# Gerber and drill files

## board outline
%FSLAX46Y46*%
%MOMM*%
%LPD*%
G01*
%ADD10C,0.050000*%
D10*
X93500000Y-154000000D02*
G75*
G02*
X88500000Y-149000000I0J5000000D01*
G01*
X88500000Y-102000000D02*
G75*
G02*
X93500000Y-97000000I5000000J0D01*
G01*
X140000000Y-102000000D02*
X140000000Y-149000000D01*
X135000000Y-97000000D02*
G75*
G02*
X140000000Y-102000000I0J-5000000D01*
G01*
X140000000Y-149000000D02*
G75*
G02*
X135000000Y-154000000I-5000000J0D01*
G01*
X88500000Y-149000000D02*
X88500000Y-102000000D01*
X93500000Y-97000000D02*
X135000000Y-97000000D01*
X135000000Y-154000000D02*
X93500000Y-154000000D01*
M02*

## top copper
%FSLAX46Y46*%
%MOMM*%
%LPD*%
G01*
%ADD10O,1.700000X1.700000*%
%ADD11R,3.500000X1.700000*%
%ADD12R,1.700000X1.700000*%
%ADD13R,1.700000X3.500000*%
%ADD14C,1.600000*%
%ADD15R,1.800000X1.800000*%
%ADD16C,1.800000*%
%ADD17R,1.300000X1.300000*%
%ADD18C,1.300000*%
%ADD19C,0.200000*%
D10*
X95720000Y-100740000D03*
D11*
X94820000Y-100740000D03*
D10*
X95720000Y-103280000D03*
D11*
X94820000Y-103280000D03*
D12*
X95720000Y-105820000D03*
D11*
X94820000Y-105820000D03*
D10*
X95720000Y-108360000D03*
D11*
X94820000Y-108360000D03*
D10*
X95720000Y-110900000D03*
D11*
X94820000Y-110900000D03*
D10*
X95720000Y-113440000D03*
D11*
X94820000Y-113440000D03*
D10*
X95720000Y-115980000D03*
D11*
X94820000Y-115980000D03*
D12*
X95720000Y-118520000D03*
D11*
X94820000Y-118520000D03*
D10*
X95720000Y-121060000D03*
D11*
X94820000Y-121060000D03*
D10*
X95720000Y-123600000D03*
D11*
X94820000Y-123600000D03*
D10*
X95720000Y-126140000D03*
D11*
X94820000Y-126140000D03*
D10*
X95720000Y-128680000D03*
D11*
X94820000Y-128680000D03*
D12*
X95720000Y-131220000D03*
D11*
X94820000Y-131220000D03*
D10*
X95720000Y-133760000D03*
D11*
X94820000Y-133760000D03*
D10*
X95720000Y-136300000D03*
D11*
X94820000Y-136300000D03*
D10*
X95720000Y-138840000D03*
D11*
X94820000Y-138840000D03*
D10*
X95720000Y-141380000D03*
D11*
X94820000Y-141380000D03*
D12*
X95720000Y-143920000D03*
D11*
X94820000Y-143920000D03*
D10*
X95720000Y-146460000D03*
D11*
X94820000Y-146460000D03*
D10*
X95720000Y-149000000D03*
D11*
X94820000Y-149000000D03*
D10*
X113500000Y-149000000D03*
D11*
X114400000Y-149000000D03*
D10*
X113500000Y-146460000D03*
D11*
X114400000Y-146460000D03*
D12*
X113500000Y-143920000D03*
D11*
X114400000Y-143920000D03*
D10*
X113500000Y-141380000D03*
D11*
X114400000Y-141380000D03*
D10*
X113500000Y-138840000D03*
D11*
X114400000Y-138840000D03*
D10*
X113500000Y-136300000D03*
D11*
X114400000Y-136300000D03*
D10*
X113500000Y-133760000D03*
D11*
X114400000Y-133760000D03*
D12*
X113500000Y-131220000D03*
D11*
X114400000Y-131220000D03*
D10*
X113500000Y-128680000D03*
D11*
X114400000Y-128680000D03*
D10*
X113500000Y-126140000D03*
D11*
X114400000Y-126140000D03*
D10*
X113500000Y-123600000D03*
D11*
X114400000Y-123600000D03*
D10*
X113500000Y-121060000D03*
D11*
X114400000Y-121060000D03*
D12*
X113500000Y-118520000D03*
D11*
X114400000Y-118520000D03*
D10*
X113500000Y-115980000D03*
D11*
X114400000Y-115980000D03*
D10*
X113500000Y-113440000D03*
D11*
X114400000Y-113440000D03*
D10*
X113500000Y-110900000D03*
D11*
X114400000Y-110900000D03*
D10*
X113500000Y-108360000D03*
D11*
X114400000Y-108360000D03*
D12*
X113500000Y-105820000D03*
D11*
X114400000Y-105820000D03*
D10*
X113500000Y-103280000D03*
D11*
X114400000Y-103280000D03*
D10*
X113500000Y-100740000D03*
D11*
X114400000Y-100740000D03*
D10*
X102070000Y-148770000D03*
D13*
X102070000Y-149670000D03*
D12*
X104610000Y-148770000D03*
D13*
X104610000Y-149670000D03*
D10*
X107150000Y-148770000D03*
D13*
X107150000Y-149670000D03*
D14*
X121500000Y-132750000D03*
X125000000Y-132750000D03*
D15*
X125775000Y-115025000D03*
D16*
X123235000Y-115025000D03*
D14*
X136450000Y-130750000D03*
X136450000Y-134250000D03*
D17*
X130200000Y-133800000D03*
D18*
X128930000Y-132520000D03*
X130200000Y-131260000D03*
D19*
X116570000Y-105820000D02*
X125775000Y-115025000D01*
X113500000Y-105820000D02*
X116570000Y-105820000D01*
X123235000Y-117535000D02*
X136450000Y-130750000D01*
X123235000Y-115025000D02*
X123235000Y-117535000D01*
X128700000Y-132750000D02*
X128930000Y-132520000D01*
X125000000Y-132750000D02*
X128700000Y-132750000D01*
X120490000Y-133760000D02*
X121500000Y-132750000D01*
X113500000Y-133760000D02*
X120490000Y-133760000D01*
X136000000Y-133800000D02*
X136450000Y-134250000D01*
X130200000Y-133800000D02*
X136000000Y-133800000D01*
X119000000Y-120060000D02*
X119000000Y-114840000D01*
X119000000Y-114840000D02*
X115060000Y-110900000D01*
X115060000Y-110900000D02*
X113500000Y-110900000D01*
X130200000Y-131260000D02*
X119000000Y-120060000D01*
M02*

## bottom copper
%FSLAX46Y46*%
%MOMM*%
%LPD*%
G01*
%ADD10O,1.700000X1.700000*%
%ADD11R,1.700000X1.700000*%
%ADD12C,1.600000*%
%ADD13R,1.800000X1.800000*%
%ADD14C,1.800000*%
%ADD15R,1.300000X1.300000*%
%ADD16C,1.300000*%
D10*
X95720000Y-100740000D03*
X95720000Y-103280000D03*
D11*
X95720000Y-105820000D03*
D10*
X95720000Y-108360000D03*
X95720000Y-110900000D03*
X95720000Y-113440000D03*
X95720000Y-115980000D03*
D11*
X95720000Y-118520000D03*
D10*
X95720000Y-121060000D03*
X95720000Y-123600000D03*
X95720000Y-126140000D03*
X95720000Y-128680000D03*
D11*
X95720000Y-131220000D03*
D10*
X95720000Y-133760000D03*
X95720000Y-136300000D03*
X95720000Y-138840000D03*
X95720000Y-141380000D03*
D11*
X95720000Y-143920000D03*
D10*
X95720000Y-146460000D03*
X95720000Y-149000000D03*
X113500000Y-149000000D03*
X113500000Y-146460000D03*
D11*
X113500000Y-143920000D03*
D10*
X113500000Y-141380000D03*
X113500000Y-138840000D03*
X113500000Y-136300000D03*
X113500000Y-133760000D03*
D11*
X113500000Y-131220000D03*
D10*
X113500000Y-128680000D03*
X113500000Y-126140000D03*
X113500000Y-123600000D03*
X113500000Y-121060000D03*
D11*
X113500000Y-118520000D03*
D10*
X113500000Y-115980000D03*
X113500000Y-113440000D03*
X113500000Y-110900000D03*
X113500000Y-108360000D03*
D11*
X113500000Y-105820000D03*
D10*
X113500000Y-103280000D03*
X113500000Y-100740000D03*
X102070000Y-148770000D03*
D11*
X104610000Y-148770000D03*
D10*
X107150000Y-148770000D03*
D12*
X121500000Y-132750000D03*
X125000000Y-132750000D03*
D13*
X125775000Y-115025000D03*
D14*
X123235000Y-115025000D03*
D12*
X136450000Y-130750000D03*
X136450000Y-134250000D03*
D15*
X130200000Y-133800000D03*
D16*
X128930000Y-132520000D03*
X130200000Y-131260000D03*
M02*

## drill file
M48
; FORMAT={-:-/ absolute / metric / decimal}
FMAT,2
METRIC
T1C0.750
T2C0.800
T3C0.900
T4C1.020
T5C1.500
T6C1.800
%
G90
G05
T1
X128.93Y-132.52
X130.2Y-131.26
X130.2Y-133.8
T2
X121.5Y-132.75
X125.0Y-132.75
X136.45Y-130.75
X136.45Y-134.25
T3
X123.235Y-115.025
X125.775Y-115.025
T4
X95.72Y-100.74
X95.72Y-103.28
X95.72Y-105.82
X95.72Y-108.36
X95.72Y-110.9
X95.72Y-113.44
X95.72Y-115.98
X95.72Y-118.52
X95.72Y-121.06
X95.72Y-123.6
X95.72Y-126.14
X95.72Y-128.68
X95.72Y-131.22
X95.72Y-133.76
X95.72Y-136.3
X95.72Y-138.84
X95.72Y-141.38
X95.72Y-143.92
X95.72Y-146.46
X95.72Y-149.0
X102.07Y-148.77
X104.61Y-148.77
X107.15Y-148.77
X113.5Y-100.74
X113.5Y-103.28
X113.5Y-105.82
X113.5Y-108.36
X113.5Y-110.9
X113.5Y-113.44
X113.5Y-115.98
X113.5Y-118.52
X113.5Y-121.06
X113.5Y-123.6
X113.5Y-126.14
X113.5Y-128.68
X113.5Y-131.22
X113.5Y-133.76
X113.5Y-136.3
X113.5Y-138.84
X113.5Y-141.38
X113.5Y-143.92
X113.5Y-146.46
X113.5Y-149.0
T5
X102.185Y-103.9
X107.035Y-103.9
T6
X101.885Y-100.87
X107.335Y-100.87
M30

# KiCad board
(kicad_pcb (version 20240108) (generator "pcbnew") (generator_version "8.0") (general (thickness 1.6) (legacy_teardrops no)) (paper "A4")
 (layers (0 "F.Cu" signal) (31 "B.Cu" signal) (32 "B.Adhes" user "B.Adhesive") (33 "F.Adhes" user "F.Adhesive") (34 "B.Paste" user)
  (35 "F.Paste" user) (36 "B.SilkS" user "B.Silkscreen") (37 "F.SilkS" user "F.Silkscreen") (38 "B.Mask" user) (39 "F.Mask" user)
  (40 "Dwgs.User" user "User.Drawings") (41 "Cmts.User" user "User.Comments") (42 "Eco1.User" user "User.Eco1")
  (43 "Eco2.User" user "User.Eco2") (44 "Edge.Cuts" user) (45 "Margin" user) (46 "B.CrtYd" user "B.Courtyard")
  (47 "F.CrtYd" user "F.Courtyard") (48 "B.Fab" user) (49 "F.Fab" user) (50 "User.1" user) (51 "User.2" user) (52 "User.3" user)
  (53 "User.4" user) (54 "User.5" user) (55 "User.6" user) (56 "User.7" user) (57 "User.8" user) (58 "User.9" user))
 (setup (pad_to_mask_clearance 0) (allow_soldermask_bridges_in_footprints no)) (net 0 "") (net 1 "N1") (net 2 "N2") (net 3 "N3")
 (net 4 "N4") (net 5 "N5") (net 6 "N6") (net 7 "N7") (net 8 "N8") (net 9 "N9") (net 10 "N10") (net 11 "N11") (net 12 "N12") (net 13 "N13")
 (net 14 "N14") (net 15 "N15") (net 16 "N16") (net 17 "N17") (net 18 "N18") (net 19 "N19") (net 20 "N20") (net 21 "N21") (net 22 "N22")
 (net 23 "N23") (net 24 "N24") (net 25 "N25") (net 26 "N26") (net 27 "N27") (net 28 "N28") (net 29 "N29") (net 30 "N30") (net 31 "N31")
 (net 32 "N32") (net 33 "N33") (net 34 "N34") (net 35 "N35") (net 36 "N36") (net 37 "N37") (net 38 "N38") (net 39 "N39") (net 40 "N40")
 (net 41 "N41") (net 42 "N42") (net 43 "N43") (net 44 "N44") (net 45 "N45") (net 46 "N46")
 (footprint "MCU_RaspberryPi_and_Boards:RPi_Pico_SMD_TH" (layer "F.Cu") (at 104.61 124.87)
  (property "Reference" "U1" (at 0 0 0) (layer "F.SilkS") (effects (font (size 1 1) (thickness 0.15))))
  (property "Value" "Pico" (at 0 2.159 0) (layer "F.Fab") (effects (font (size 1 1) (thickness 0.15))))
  (pad "" np_thru_hole oval (at -2.725 -24) (size 1.8 1.8) (drill 1.8) (layers "*.Cu" "*.Mask"))
  (pad "" np_thru_hole oval (at -2.425 -20.97) (size 1.5 1.5) (drill 1.5) (layers "*.Cu" "*.Mask"))
  (pad "" np_thru_hole oval (at 2.425 -20.97) (size 1.5 1.5) (drill 1.5) (layers "*.Cu" "*.Mask"))
  (pad "" np_thru_hole oval (at 2.725 -24) (size 1.8 1.8) (drill 1.8) (layers "*.Cu" "*.Mask"))
  (pad "1" thru_hole oval (at -8.89 -24.13) (size 1.7 1.7) (drill 1.02) (layers "*.Cu" "*.Mask") (remove_unused_layers no) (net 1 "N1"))
  (pad "1" smd rect (at -8.89 -24.13) (size 3.5 1.7) (drill (offset -0.9 0)) (layers "F.Cu" "F.Mask") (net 1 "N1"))
  (pad "2" thru_hole oval (at -8.89 -21.59) (size 1.7 1.7) (drill 1.02) (layers "*.Cu" "*.Mask") (remove_unused_layers no) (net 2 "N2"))
  (pad "2" smd rect (at -8.89 -21.59) (size 3.5 1.7) (drill (offset -0.9 0)) (layers "F.Cu" "F.Mask") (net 2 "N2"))
  (pad "3" thru_hole rect (at -8.89 -19.05) (size 1.7 1.7) (drill 1.02) (layers "*.Cu" "*.Mask") (remove_unused_layers no) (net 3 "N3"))
  (pad "3" smd rect (at -8.89 -19.05) (size 3.5 1.7) (drill (offset -0.9 0)) (layers "F.Cu" "F.Mask") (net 3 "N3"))
  (pad "4" thru_hole oval (at -8.89 -16.51) (size 1.7 1.7) (drill 1.02) (layers "*.Cu" "*.Mask") (remove_unused_layers no) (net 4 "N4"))
  (pad "4" smd rect (at -8.89 -16.51) (size 3.5 1.7) (drill (offset -0.9 0)) (layers "F.Cu" "F.Mask") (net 4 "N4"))
  (pad "5" thru_hole oval (at -8.89 -13.97) (size 1.7 1.7) (drill 1.02) (layers "*.Cu" "*.Mask") (remove_unused_layers no) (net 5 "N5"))
  (pad "5" smd rect (at -8.89 -13.97) (size 3.5 1.7) (drill (offset -0.9 0)) (layers "F.Cu" "F.Mask") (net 5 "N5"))
  (pad "6" thru_hole oval (at -8.89 -11.43) (size 1.7 1.7) (drill 1.02) (layers "*.Cu" "*.Mask") (remove_unused_layers no) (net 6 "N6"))
  (pad "6" smd rect (at -8.89 -11.43) (size 3.5 1.7) (drill (offset -0.9 0)) (layers "F.Cu" "F.Mask") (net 6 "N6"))
  (pad "7" thru_hole oval (at -8.89 -8.89) (size 1.7 1.7) (drill 1.02) (layers "*.Cu" "*.Mask") (remove_unused_layers no) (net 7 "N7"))
  (pad "7" smd rect (at -8.89 -8.89) (size 3.5 1.7) (drill (offset -0.9 0)) (layers "F.Cu" "F.Mask") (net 7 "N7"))
  (pad "8" thru_hole rect (at -8.89 -6.35) (size 1.7 1.7) (drill 1.02) (layers "*.Cu" "*.Mask") (remove_unused_layers no) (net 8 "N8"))
  (pad "8" smd rect (at -8.89 -6.35) (size 3.5 1.7) (drill (offset -0.9 0)) (layers "F.Cu" "F.Mask") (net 8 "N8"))
  (pad "9" thru_hole oval (at -8.89 -3.81) (size 1.7 1.7) (drill 1.02) (layers "*.Cu" "*.Mask") (remove_unused_layers no) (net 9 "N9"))
  (pad "9" smd rect (at -8.89 -3.81) (size 3.5 1.7) (drill (offset -0.9 0)) (layers "F.Cu" "F.Mask") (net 9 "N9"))
  (pad "10" thru_hole oval (at -8.89 -1.27) (size 1.7 1.7) (drill 1.02) (layers "*.Cu" "*.Mask") (remove_unused_layers no) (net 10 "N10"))
  (pad "10" smd rect (at -8.89 -1.27) (size 3.5 1.7) (drill (offset -0.9 0)) (layers "F.Cu" "F.Mask") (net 10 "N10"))
  (pad "11" thru_hole oval (at -8.89 1.27) (size 1.7 1.7) (drill 1.02) (layers "*.Cu" "*.Mask") (remove_unused_layers no) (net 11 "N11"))
  (pad "11" smd rect (at -8.89 1.27) (size 3.5 1.7) (drill (offset -0.9 0)) (layers "F.Cu" "F.Mask") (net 11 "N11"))
  (pad "12" thru_hole oval (at -8.89 3.81) (size 1.7 1.7) (drill 1.02) (layers "*.Cu" "*.Mask") (remove_unused_layers no) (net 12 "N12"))
  (pad "12" smd rect (at -8.89 3.81) (size 3.5 1.7) (drill (offset -0.9 0)) (layers "F.Cu" "F.Mask") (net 12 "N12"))
  (pad "13" thru_hole rect (at -8.89 6.35) (size 1.7 1.7) (drill 1.02) (layers "*.Cu" "*.Mask") (remove_unused_layers no) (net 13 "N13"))
  (pad "13" smd rect (at -8.89 6.35) (size 3.5 1.7) (drill (offset -0.9 0)) (layers "F.Cu" "F.Mask") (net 13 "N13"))
  (pad "14" thru_hole oval (at -8.89 8.89) (size 1.7 1.7) (drill 1.02) (layers "*.Cu" "*.Mask") (remove_unused_layers no) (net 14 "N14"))
  (pad "14" smd rect (at -8.89 8.89) (size 3.5 1.7) (drill (offset -0.9 0)) (layers "F.Cu" "F.Mask") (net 14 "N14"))
  (pad "15" thru_hole oval (at -8.89 11.43) (size 1.7 1.7) (drill 1.02) (layers "*.Cu" "*.Mask") (remove_unused_layers no) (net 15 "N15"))
  (pad "15" smd rect (at -8.89 11.43) (size 3.5 1.7) (drill (offset -0.9 0)) (layers "F.Cu" "F.Mask") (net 15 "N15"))
  (pad "16" thru_hole oval (at -8.89 13.97) (size 1.7 1.7) (drill 1.02) (layers "*.Cu" "*.Mask") (remove_unused_layers no) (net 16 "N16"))
  (pad "16" smd rect (at -8.89 13.97) (size 3.5 1.7) (drill (offset -0.9 0)) (layers "F.Cu" "F.Mask") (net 16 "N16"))
  (pad "17" thru_hole oval (at -8.89 16.51) (size 1.7 1.7) (drill 1.02) (layers "*.Cu" "*.Mask") (remove_unused_layers no) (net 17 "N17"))
  (pad "17" smd rect (at -8.89 16.51) (size 3.5 1.7) (drill (offset -0.9 0)) (layers "F.Cu" "F.Mask") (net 17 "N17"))
  (pad "18" thru_hole rect (at -8.89 19.05) (size 1.7 1.7) (drill 1.02) (layers "*.Cu" "*.Mask") (remove_unused_layers no) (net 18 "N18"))
  (pad "18" smd rect (at -8.89 19.05) (size 3.5 1.7) (drill (offset -0.9 0)) (layers "F.Cu" "F.Mask") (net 18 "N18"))
  (pad "19" thru_hole oval (at -8.89 21.59) (size 1.7 1.7) (drill 1.02) (layers "*.Cu" "*.Mask") (remove_unused_layers no) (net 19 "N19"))
  (pad "19" smd rect (at -8.89 21.59) (size 3.5 1.7) (drill (offset -0.9 0)) (layers "F.Cu" "F.Mask") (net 19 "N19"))
  (pad "20" thru_hole oval (at -8.89 24.13) (size 1.7 1.7) (drill 1.02) (layers "*.Cu" "*.Mask") (remove_unused_layers no) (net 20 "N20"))
  (pad "20" smd rect (at -8.89 24.13) (size 3.5 1.7) (drill (offset -0.9 0)) (layers "F.Cu" "F.Mask") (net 20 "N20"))
  (pad "21" thru_hole oval (at 8.89 24.13) (size 1.7 1.7) (drill 1.02) (layers "*.Cu" "*.Mask") (remove_unused_layers no) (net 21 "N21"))
  (pad "21" smd rect (at 8.89 24.13) (size 3.5 1.7) (drill (offset 0.9 0)) (layers "F.Cu" "F.Mask") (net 21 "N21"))
  (pad "22" thru_hole oval (at 8.89 21.59) (size 1.7 1.7) (drill 1.02) (layers "*.Cu" "*.Mask") (remove_unused_layers no) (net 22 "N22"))
  (pad "22" smd rect (at 8.89 21.59) (size 3.5 1.7) (drill (offset 0.9 0)) (layers "F.Cu" "F.Mask") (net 22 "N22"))
  (pad "23" thru_hole rect (at 8.89 19.05) (size 1.7 1.7) (drill 1.02) (layers "*.Cu" "*.Mask") (remove_unused_layers no) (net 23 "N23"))
  (pad "23" smd rect (at 8.89 19.05) (size 3.5 1.7) (drill (offset 0.9 0)) (layers "F.Cu" "F.Mask") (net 23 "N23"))
  (pad "24" thru_hole oval (at 8.89 16.51) (size 1.7 1.7) (drill 1.02) (layers "*.Cu" "*.Mask") (remove_unused_layers no) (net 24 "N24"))
  (pad "24" smd rect (at 8.89 16.51) (size 3.5 1.7) (drill (offset 0.9 0)) (layers "F.Cu" "F.Mask") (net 24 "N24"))
  (pad "25" thru_hole oval (at 8.89 13.97) (size 1.7 1.7) (drill 1.02) (layers "*.Cu" "*.Mask") (remove_unused_layers no) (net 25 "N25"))
  (pad "25" smd rect (at 8.89 13.97) (size 3.5 1.7) (drill (offset 0.9 0)) (layers "F.Cu" "F.Mask") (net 25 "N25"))
  (pad "26" thru_hole oval (at 8.89 11.43) (size 1.7 1.7) (drill 1.02) (layers "*.Cu" "*.Mask") (remove_unused_layers no) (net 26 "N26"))
  (pad "26" smd rect (at 8.89 11.43) (size 3.5 1.7) (drill (offset 0.9 0)) (layers "F.Cu" "F.Mask") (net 26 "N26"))
  (pad "27" thru_hole oval (at 8.89 8.89) (size 1.7 1.7) (drill 1.02) (layers "*.Cu" "*.Mask") (remove_unused_layers no) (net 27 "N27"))
  (pad "27" smd rect (at 8.89 8.89) (size 3.5 1.7) (drill (offset 0.9 0)) (layers "F.Cu" "F.Mask") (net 27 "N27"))
  (pad "28" thru_hole rect (at 8.89 6.35) (size 1.7 1.7) (drill 1.02) (layers "*.Cu" "*.Mask") (remove_unused_layers no) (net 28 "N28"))
  (pad "28" smd rect (at 8.89 6.35) (size 3.5 1.7) (drill (offset 0.9 0)) (layers "F.Cu" "F.Mask") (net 28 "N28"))
  (pad "29" thru_hole oval (at 8.89 3.81) (size 1.7 1.7) (drill 1.02) (layers "*.Cu" "*.Mask") (remove_unused_layers no) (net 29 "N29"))
  (pad "29" smd rect (at 8.89 3.81) (size 3.5 1.7) (drill (offset 0.9 0)) (layers "F.Cu" "F.Mask") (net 29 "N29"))
  (pad "30" thru_hole oval (at 8.89 1.27) (size 1.7 1.7) (drill 1.02) (layers "*.Cu" "*.Mask") (remove_unused_layers no) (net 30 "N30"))
  (pad "30" smd rect (at 8.89 1.27) (size 3.5 1.7) (drill (offset 0.9 0)) (layers "F.Cu" "F.Mask") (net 30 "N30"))
  (pad "31" thru_hole oval (at 8.89 -1.27) (size 1.7 1.7) (drill 1.02) (layers "*.Cu" "*.Mask") (remove_unused_layers no) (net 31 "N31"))
  (pad "31" smd rect (at 8.89 -1.27) (size 3.5 1.7) (drill (offset 0.9 0)) (layers "F.Cu" "F.Mask") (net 31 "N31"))
  (pad "32" thru_hole oval (at 8.89 -3.81) (size 1.7 1.7) (drill 1.02) (layers "*.Cu" "*.Mask") (remove_unused_layers no) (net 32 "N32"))
  (pad "32" smd rect (at 8.89 -3.81) (size 3.5 1.7) (drill (offset 0.9 0)) (layers "F.Cu" "F.Mask") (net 32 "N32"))
  (pad "33" thru_hole rect (at 8.89 -6.35) (size 1.7 1.7) (drill 1.02) (layers "*.Cu" "*.Mask") (remove_unused_layers no) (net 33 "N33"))
  (pad "33" smd rect (at 8.89 -6.35) (size 3.5 1.7) (drill (offset 0.9 0)) (layers "F.Cu" "F.Mask") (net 33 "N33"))
  (pad "34" thru_hole oval (at 8.89 -8.89) (size 1.7 1.7) (drill 1.02) (layers "*.Cu" "*.Mask") (remove_unused_layers no) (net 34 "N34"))
  (pad "34" smd rect (at 8.89 -8.89) (size 3.5 1.7) (drill (offset 0.9 0)) (layers "F.Cu" "F.Mask") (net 34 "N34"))
  (pad "35" thru_hole oval (at 8.89 -11.43) (size 1.7 1.7) (drill 1.02) (layers "*.Cu" "*.Mask") (remove_unused_layers no) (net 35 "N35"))
  (pad "35" smd rect (at 8.89 -11.43) (size 3.5 1.7) (drill (offset 0.9 0)) (layers "F.Cu" "F.Mask") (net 35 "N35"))
  (pad "36" thru_hole oval (at 8.89 -13.97) (size 1.7 1.7) (drill 1.02) (layers "*.Cu" "*.Mask") (remove_unused_layers no) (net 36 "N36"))
  (pad "36" smd rect (at 8.89 -13.97) (size 3.5 1.7) (drill (offset 0.9 0)) (layers "F.Cu" "F.Mask") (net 36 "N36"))
  (pad "37" thru_hole oval (at 8.89 -16.51) (size 1.7 1.7) (drill 1.02) (layers "*.Cu" "*.Mask") (remove_unused_layers no) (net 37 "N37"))
  (pad "37" smd rect (at 8.89 -16.51) (size 3.5 1.7) (drill (offset 0.9 0)) (layers "F.Cu" "F.Mask") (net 37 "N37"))
  (pad "38" thru_hole rect (at 8.89 -19.05) (size 1.7 1.7) (drill 1.02) (layers "*.Cu" "*.Mask") (remove_unused_layers no) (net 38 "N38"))
  (pad "38" smd rect (at 8.89 -19.05) (size 3.5 1.7) (drill (offset 0.9 0)) (layers "F.Cu" "F.Mask") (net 38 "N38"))
  (pad "39" thru_hole oval (at 8.89 -21.59) (size 1.7 1.7) (drill 1.02) (layers "*.Cu" "*.Mask") (remove_unused_layers no) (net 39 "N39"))
  (pad "39" smd rect (at 8.89 -21.59) (size 3.5 1.7) (drill (offset 0.9 0)) (layers "F.Cu" "F.Mask") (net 39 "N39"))
  (pad "40" thru_hole oval (at 8.89 -24.13) (size 1.7 1.7) (drill 1.02) (layers "*.Cu" "*.Mask") (remove_unused_layers no) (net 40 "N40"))
  (pad "40" smd rect (at 8.89 -24.13) (size 3.5 1.7) (drill (offset 0.9 0)) (layers "F.Cu" "F.Mask") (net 40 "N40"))
  (pad "41" thru_hole oval (at -2.54 23.9) (size 1.7 1.7) (drill 1.02) (layers "*.Cu" "*.Mask") (remove_unused_layers no) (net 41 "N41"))
  (pad "41" smd rect (at -2.54 23.9 90) (size 3.5 1.7) (drill (offset -0.9 0)) (layers "F.Cu" "F.Mask") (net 41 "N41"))
  (pad "42" thru_hole rect (at 0 23.9) (size 1.7 1.7) (drill 1.02) (layers "*.Cu" "*.Mask") (remove_unused_layers no) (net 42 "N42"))
  (pad "42" smd rect (at 0 23.9 90) (size 3.5 1.7) (drill (offset -0.9 0)) (layers "F.Cu" "F.Mask") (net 42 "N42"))
  (pad "43" thru_hole oval (at 2.54 23.9) (size 1.7 1.7) (drill 1.02) (layers "*.Cu" "*.Mask") (remove_unused_layers no) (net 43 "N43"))
  (pad "43" smd rect (at 2.54 23.9 90) (size 3.5 1.7) (drill (offset -0.9 0)) (layers "F.Cu" "F.Mask") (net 43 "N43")))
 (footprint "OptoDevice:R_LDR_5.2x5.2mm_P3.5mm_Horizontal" (layer "F.Cu") (at 121.5 132.75)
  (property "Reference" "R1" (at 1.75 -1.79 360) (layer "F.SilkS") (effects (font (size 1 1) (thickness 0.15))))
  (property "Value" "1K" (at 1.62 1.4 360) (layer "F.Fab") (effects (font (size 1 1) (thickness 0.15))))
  (pad "1" thru_hole circle (at 0 0) (size 1.6 1.6) (drill 0.8) (layers "*.Cu" "*.Mask") (remove_unused_layers no) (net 27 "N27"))
  (pad "2" thru_hole circle (at 3.5 0) (size 1.6 1.6) (drill 0.8) (layers "*.Cu" "*.Mask") (remove_unused_layers no) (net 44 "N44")))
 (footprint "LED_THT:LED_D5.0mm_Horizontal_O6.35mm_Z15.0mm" (layer "F.Cu") (at 125.775 115.025 180)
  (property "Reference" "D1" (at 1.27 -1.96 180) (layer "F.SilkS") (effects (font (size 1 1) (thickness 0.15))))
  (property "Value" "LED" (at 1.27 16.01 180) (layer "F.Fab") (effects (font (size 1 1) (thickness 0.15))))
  (pad "1" thru_hole rect (at 0 0 180) (size 1.8 1.8) (drill 0.9) (layers "*.Cu" "*.Mask") (remove_unused_layers no) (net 38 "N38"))
  (pad "2" thru_hole circle (at 2.54 0 180) (size 1.8 1.8) (drill 0.9) (layers "*.Cu" "*.Mask") (remove_unused_layers no) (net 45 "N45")))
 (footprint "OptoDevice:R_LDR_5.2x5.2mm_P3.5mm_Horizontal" (layer "F.Cu") (at 136.45 130.75 -90)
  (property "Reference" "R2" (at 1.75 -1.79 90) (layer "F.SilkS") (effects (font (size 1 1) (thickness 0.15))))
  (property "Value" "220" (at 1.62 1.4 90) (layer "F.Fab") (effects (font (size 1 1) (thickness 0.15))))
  (pad "1" thru_hole circle (at 0 0 270) (size 1.6 1.6) (drill 0.8) (layers "*.Cu" "*.Mask") (remove_unused_layers no) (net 45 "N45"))
  (pad "2" thru_hole circle (at 3.5 0 270) (size 1.6 1.6) (drill 0.8) (layers "*.Cu" "*.Mask") (remove_unused_layers no) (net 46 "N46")))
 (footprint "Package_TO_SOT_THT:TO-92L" (layer "F.Cu") (at 130.2 133.8 90)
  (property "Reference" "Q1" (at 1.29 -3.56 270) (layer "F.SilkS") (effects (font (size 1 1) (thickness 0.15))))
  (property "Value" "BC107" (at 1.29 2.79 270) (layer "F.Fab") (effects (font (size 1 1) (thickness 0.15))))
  (pad "1" thru_hole rect (at 0 0 90) (size 1.3 1.3) (drill 0.75) (layers "*.Cu" "*.Mask") (remove_unused_layers no) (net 46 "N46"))
  (pad "2" thru_hole circle (at 1.28 -1.27 90) (size 1.3 1.3) (drill 0.75) (layers "*.Cu" "*.Mask") (remove_unused_layers no) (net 44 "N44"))
  (pad "3" thru_hole circle (at 2.54 0 90) (size 1.3 1.3) (drill 0.75) (layers "*.Cu" "*.Mask") (remove_unused_layers no) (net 36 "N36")))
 (gr_arc (start 93.5 154) (mid 89.964466 152.535534) (end 88.5 149) (stroke (width 0.05) (type default)) (layer "Edge.Cuts"))
 (gr_arc (start 88.5 102) (mid 89.964466 98.464466) (end 93.5 97) (stroke (width 0.05) (type default)) (layer "Edge.Cuts"))
 (gr_line (start 140 102) (end 140 149) (stroke (width 0.05) (type default)) (layer "Edge.Cuts"))
 (gr_arc (start 135 97) (mid 138.535534 98.464466) (end 140 102) (stroke (width 0.05) (type default)) (layer "Edge.Cuts"))
 (gr_arc (start 140 149) (mid 138.535534 152.535534) (end 135 154) (stroke (width 0.05) (type default)) (layer "Edge.Cuts"))
 (gr_line (start 88.5 149) (end 88.5 102) (stroke (width 0.05) (type default)) (layer "Edge.Cuts"))
 (gr_line (start 93.5 97) (end 135 97) (stroke (width 0.05) (type default)) (layer "Edge.Cuts"))
 (gr_line (start 135 154) (end 93.5 154) (stroke (width 0.05) (type default)) (layer "Edge.Cuts"))
 (segment (start 116.57 105.82) (end 125.775 115.025) (width 0.2) (layer "F.Cu") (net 38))
 (segment (start 113.5 105.82) (end 116.57 105.82) (width 0.2) (layer "F.Cu") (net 38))
 (segment (start 123.235 117.535) (end 136.45 130.75) (width 0.2) (layer "F.Cu") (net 45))
 (segment (start 123.235 115.025) (end 123.235 117.535) (width 0.2) (layer "F.Cu") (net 45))
 (segment (start 128.7 132.75) (end 128.93 132.52) (width 0.2) (layer "F.Cu") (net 44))
 (segment (start 125 132.75) (end 128.7 132.75) (width 0.2) (layer "F.Cu") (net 44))
 (segment (start 120.49 133.76) (end 121.5 132.75) (width 0.2) (layer "F.Cu") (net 27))
 (segment (start 113.5 133.76) (end 120.49 133.76) (width 0.2) (layer "F.Cu") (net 27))
 (segment (start 136 133.8) (end 136.45 134.25) (width 0.2) (layer "F.Cu") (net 46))
 (segment (start 130.2 133.8) (end 136 133.8) (width 0.2) (layer "F.Cu") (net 46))
 (segment (start 119 120.06) (end 119 114.84) (width 0.2) (layer "F.Cu") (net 36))
 (segment (start 119 114.84) (end 115.06 110.9) (width 0.2) (layer "F.Cu") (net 36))
 (segment (start 115.06 110.9) (end 113.5 110.9) (width 0.2) (layer "F.Cu") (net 36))
 (segment (start 130.2 131.26) (end 119 120.06) (width 0.2) (layer "F.Cu") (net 36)))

